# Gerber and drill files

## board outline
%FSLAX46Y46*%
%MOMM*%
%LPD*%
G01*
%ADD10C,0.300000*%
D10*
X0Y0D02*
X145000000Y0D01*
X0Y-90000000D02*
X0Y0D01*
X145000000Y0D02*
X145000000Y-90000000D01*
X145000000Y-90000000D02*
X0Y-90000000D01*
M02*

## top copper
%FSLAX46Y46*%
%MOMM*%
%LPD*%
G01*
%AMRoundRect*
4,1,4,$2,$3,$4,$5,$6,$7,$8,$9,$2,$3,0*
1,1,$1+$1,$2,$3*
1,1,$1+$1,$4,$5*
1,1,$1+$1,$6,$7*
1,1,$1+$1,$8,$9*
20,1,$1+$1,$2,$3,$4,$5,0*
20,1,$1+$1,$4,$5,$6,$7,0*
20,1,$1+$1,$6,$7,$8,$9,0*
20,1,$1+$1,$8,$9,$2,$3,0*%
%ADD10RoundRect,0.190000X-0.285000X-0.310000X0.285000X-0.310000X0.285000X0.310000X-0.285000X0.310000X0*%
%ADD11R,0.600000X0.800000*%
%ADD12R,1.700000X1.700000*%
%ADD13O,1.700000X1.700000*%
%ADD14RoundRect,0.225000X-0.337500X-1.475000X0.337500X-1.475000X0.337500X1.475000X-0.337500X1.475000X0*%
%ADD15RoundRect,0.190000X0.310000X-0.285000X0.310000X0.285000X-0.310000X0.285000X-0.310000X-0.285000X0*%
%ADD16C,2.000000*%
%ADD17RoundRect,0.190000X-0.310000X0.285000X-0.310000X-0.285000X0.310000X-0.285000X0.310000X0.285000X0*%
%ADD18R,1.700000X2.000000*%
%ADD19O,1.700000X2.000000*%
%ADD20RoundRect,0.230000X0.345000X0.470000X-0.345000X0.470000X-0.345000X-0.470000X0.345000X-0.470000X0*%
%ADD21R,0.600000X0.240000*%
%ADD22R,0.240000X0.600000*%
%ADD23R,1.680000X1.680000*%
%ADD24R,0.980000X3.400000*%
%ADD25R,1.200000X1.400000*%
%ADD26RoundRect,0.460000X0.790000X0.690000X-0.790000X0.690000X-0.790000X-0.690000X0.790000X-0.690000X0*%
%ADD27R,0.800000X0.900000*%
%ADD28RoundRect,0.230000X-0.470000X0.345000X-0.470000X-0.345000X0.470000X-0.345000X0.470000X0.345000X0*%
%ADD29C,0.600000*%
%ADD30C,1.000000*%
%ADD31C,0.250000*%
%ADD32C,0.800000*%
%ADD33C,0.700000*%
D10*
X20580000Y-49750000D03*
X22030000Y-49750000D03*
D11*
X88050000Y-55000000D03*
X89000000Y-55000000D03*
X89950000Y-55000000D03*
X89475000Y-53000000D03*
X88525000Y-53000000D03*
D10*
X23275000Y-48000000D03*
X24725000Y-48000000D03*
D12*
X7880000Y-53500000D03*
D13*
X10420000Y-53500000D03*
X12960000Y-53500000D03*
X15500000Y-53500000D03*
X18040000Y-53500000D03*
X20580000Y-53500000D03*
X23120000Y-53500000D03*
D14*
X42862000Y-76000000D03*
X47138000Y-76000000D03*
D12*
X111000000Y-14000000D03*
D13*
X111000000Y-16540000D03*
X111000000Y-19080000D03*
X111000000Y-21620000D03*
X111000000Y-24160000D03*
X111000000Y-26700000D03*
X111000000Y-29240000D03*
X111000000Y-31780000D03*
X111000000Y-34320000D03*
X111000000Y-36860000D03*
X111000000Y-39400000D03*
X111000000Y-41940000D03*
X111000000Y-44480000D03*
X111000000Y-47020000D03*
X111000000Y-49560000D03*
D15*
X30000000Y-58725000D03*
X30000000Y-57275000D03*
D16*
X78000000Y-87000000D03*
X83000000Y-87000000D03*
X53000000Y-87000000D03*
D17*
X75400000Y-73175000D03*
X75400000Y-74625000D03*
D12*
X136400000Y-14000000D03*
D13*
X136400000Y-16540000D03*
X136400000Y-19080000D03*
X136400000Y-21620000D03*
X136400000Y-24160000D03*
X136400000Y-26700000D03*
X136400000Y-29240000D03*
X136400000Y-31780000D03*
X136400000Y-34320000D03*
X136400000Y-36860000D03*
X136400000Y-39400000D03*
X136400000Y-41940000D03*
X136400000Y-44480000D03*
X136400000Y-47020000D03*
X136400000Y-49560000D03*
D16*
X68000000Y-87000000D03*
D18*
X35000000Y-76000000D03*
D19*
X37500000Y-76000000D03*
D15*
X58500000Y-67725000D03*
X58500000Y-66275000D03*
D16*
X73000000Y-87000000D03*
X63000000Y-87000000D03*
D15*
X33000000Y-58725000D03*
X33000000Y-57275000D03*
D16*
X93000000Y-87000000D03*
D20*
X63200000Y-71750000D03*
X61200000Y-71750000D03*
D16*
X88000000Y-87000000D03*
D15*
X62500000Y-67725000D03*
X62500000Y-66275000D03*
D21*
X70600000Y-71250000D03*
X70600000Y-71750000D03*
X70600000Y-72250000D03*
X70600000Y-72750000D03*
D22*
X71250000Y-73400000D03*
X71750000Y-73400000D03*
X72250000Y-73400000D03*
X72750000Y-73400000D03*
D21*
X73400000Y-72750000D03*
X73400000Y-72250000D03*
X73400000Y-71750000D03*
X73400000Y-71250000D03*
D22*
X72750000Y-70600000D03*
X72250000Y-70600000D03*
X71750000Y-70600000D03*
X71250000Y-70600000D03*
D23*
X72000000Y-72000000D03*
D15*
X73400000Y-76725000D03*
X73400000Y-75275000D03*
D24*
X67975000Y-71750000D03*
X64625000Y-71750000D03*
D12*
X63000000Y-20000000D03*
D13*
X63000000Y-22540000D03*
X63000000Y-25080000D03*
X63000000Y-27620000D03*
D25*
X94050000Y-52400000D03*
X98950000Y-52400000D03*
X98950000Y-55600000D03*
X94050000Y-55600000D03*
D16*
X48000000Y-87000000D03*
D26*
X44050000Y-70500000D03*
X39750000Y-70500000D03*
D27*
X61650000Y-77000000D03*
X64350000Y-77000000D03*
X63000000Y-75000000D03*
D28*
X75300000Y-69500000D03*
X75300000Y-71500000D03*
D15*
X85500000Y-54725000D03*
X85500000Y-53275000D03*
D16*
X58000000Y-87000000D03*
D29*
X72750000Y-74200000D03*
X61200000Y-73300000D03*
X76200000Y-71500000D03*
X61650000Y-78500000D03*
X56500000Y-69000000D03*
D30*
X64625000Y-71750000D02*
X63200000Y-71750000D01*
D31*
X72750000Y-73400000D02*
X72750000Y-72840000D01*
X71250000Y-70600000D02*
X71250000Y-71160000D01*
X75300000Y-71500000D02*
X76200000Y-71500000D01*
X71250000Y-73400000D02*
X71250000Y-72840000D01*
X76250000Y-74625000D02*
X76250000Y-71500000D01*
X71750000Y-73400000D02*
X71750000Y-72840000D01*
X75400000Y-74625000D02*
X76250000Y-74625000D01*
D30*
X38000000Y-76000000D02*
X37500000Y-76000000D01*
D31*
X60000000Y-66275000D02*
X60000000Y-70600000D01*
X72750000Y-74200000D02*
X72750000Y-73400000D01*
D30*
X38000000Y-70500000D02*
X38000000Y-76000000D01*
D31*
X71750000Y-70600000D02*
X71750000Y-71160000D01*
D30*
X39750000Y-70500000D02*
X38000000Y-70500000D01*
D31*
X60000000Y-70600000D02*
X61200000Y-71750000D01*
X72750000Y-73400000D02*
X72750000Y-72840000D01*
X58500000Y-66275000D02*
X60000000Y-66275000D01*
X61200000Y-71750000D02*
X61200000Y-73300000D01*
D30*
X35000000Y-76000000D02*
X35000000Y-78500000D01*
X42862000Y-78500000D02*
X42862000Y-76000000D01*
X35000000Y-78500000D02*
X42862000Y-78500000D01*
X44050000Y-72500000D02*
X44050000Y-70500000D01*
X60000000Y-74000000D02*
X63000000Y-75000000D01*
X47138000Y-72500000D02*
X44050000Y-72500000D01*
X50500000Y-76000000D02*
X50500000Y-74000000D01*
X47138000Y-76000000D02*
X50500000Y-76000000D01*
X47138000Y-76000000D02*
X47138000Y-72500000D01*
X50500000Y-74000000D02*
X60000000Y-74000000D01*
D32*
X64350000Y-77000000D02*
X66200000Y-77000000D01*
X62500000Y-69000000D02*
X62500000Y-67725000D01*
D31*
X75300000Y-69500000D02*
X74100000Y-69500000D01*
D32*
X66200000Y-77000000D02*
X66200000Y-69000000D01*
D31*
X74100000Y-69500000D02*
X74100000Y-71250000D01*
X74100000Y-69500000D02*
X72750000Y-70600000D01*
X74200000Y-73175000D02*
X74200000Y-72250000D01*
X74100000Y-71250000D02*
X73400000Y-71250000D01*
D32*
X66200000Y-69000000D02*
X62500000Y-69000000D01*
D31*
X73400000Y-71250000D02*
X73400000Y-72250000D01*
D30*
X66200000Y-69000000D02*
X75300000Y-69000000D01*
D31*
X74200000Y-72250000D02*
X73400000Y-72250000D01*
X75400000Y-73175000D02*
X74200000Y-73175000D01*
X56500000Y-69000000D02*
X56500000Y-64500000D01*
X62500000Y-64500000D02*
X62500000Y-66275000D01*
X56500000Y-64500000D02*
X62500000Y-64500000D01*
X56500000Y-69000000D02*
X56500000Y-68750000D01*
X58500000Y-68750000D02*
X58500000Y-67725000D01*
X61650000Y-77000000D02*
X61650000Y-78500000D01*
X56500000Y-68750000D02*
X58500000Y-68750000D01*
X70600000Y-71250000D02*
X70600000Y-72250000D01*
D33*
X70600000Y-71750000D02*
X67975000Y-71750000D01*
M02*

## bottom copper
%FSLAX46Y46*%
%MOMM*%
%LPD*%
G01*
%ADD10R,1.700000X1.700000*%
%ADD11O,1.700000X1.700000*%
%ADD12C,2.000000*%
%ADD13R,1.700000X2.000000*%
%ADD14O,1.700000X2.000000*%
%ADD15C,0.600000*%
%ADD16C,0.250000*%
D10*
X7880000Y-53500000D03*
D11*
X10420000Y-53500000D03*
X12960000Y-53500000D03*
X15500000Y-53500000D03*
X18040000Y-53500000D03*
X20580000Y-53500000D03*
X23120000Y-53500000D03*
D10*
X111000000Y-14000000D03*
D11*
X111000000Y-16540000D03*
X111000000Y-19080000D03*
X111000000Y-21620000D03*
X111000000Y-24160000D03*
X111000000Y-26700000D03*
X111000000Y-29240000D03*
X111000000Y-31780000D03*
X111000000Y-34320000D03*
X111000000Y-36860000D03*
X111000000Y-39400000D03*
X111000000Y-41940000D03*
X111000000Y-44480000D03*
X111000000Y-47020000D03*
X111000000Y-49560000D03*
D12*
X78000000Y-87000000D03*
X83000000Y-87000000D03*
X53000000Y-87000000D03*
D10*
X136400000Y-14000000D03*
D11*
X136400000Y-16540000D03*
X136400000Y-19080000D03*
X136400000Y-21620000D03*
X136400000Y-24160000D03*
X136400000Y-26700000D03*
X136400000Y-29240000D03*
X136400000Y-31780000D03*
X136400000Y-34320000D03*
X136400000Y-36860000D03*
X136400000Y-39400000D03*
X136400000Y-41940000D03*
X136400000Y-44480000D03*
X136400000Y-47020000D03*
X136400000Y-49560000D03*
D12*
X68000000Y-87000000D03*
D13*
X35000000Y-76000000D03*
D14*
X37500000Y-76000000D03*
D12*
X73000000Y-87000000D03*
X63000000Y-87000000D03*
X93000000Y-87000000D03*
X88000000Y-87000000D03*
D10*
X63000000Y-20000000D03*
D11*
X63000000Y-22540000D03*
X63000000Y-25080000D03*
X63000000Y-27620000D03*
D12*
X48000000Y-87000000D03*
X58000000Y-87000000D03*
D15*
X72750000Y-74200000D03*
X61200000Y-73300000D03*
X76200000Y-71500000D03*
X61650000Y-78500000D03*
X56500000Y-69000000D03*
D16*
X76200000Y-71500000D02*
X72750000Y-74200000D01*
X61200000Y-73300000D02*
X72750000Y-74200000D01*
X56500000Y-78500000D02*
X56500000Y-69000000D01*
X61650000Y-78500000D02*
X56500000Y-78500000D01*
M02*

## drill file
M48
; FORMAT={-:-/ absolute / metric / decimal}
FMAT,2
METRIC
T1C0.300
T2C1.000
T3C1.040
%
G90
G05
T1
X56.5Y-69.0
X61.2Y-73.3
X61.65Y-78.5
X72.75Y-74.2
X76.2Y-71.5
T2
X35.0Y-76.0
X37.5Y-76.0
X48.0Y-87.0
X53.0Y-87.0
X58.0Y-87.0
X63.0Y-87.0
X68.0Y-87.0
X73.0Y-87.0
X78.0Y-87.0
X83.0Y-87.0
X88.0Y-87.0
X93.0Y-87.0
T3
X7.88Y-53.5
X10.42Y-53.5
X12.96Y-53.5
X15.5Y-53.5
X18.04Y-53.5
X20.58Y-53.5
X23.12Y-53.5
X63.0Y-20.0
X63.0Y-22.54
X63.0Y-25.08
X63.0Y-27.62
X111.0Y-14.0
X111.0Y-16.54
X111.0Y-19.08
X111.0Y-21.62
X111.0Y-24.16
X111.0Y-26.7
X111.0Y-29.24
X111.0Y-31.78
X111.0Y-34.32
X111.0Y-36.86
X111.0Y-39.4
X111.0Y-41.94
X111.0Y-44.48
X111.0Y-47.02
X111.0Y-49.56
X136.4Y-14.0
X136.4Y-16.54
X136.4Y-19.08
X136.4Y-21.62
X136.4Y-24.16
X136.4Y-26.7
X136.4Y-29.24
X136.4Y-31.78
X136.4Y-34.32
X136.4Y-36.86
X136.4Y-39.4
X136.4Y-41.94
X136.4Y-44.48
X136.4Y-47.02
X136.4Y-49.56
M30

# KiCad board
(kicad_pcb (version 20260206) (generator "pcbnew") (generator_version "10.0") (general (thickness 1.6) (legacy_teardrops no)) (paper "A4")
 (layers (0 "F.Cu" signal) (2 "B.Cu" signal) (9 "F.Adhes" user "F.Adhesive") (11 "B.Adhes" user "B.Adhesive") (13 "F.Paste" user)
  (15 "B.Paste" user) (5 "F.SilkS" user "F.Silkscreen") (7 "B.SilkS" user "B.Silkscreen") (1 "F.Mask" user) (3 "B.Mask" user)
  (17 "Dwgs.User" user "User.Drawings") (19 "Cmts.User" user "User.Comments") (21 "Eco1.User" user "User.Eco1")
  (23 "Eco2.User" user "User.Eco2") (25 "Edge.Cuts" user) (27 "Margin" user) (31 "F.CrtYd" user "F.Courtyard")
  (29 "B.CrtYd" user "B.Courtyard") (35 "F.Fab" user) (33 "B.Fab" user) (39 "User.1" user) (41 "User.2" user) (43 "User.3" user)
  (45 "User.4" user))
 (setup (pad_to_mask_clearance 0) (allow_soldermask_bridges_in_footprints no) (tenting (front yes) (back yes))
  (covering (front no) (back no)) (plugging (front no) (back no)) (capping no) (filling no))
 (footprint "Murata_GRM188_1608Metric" (layer "F.Cu") (at 21.305 49.75)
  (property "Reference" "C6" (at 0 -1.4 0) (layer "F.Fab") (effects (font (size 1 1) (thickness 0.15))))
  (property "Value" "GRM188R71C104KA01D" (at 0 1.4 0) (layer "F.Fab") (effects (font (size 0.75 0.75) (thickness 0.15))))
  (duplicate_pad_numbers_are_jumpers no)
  (pad "1" smd roundrect (at -0.725 0) (size 0.95 1) (layers "F.Cu" "F.Mask" "F.Paste") (roundrect_rratio 0.2) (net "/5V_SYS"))
  (pad "2" smd roundrect (at 0.725 0) (size 0.95 1) (layers "F.Cu" "F.Mask" "F.Paste") (roundrect_rratio 0.2) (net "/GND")))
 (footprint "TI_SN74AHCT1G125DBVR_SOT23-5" (layer "F.Cu") (at 89 54)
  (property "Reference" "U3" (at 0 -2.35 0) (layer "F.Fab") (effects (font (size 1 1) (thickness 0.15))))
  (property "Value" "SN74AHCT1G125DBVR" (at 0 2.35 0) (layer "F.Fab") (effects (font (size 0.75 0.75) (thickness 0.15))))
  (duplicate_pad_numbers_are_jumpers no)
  (pad "1" smd rect (at -0.95 1) (size 0.6 0.8) (layers "F.Cu" "F.Mask" "F.Paste") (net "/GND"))
  (pad "2" smd rect (at 0 1) (size 0.6 0.8) (layers "F.Cu" "F.Mask" "F.Paste") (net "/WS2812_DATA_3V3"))
  (pad "3" smd rect (at 0.95 1) (size 0.6 0.8) (layers "F.Cu" "F.Mask" "F.Paste") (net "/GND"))
  (pad "4" smd rect (at 0.475 -1) (size 0.6 0.8) (layers "F.Cu" "F.Mask" "F.Paste") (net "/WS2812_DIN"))
  (pad "5" smd rect (at -0.475 -1) (size 0.6 0.8) (layers "F.Cu" "F.Mask" "F.Paste") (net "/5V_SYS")))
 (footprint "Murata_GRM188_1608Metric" (layer "F.Cu") (at 24 48)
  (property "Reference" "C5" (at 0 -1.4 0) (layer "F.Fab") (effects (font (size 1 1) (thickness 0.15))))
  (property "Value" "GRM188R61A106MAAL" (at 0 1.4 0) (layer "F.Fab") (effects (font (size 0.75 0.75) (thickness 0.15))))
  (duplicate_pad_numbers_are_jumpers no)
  (pad "1" smd roundrect (at -0.725 0) (size 0.95 1) (layers "F.Cu" "F.Mask" "F.Paste") (roundrect_rratio 0.2) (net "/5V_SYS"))
  (pad "2" smd roundrect (at 0.725 0) (size 0.95 1) (layers "F.Cu" "F.Mask" "F.Paste") (roundrect_rratio 0.2) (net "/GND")))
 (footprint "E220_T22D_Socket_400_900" (layer "F.Cu") (at 5 52)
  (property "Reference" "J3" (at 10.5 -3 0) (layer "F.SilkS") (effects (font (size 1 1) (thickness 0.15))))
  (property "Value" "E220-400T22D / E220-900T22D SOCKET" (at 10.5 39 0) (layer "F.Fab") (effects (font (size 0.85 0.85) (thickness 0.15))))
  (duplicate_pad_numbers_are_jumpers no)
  (pad "1" thru_hole rect (at 2.88 1.5) (size 1.7 1.7) (drill 1.04) (layers "*.Cu" "*.Mask") (remove_unused_layers no) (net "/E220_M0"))
  (pad "2" thru_hole oval (at 5.42 1.5) (size 1.7 1.7) (drill 1.04) (layers "*.Cu" "*.Mask") (remove_unused_layers no) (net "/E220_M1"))
  (pad "3" thru_hole oval (at 7.96 1.5) (size 1.7 1.7) (drill 1.04) (layers "*.Cu" "*.Mask") (remove_unused_layers no) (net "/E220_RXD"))
  (pad "4" thru_hole oval (at 10.5 1.5) (size 1.7 1.7) (drill 1.04) (layers "*.Cu" "*.Mask") (remove_unused_layers no) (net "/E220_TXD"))
  (pad "5" thru_hole oval (at 13.04 1.5) (size 1.7 1.7) (drill 1.04) (layers "*.Cu" "*.Mask") (remove_unused_layers no) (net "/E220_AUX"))
  (pad "6" thru_hole oval (at 15.58 1.5) (size 1.7 1.7) (drill 1.04) (layers "*.Cu" "*.Mask") (remove_unused_layers no) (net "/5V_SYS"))
  (pad "7" thru_hole oval (at 18.12 1.5) (size 1.7 1.7) (drill 1.04) (layers "*.Cu" "*.Mask") (remove_unused_layers no) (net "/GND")))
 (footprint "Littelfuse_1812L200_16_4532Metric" (layer "F.Cu") (at 45 76)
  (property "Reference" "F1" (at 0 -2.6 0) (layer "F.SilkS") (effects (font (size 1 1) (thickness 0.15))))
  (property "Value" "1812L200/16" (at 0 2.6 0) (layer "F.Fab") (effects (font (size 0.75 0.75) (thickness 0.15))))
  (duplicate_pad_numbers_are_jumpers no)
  (pad "1" smd roundrect (at -2.138 0) (size 1.125 3.4) (layers "F.Cu" "F.Mask" "F.Paste") (roundrect_rratio 0.2) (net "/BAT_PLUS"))
  (pad "2" smd roundrect (at 2.138 0) (size 1.125 3.4) (layers "F.Cu" "F.Mask" "F.Paste") (roundrect_rratio 0.2) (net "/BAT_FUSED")))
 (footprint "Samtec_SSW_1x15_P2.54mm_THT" (layer "F.Cu") (at 111 14)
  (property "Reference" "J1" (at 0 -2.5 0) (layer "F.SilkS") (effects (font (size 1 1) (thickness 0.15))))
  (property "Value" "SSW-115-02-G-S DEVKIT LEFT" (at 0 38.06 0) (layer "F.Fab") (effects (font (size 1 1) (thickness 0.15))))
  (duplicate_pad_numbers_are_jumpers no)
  (pad "1" thru_hole rect (at 0 0) (size 1.7 1.7) (drill 1.04) (layers "*.Cu" "*.Mask") (remove_unused_layers no) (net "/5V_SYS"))
  (pad "2" thru_hole oval (at 0 2.54) (size 1.7 1.7) (drill 1.04) (layers "*.Cu" "*.Mask") (remove_unused_layers no) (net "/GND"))
  (pad "3" thru_hole oval (at 0 5.08) (size 1.7 1.7) (drill 1.04) (layers "*.Cu" "*.Mask") (remove_unused_layers no))
  (pad "4" thru_hole oval (at 0 7.62) (size 1.7 1.7) (drill 1.04) (layers "*.Cu" "*.Mask") (remove_unused_layers no))
  (pad "5" thru_hole oval (at 0 10.16) (size 1.7 1.7) (drill 1.04) (layers "*.Cu" "*.Mask") (remove_unused_layers no))
  (pad "6" thru_hole oval (at 0 12.7) (size 1.7 1.7) (drill 1.04) (layers "*.Cu" "*.Mask") (remove_unused_layers no) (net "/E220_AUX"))
  (pad "7" thru_hole oval (at 0 15.24) (size 1.7 1.7) (drill 1.04) (layers "*.Cu" "*.Mask") (remove_unused_layers no) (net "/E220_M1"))
  (pad "8" thru_hole oval (at 0 17.78) (size 1.7 1.7) (drill 1.04) (layers "*.Cu" "*.Mask") (remove_unused_layers no) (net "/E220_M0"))
  (pad "9" thru_hole oval (at 0 20.32) (size 1.7 1.7) (drill 1.04) (layers "*.Cu" "*.Mask") (remove_unused_layers no))
  (pad "10" thru_hole oval (at 0 22.86) (size 1.7 1.7) (drill 1.04) (layers "*.Cu" "*.Mask") (remove_unused_layers no))
  (pad "11" thru_hole oval (at 0 25.4) (size 1.7 1.7) (drill 1.04) (layers "*.Cu" "*.Mask") (remove_unused_layers no))
  (pad "12" thru_hole oval (at 0 27.94) (size 1.7 1.7) (drill 1.04) (layers "*.Cu" "*.Mask") (remove_unused_layers no))
  (pad "13" thru_hole oval (at 0 30.48) (size 1.7 1.7) (drill 1.04) (layers "*.Cu" "*.Mask") (remove_unused_layers no))
  (pad "14" thru_hole oval (at 0 33.02) (size 1.7 1.7) (drill 1.04) (layers "*.Cu" "*.Mask") (remove_unused_layers no))
  (pad "15" thru_hole oval (at 0 35.56) (size 1.7 1.7) (drill 1.04) (layers "*.Cu" "*.Mask") (remove_unused_layers no)))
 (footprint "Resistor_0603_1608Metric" (layer "F.Cu") (at 30 58 90)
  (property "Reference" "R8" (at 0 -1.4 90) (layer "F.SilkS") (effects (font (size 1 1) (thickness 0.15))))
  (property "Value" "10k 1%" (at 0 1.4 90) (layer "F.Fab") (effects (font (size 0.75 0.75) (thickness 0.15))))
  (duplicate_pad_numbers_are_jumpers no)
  (pad "1" smd roundrect (at -0.725 0 90) (size 0.95 1) (layers "F.Cu" "F.Mask" "F.Paste") (roundrect_rratio 0.2) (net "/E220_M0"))
  (pad "2" smd roundrect (at 0.725 0 90) (size 0.95 1) (layers "F.Cu" "F.Mask" "F.Paste") (roundrect_rratio 0.2) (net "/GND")))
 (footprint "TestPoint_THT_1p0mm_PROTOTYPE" (layer "F.Cu") (at 78 87)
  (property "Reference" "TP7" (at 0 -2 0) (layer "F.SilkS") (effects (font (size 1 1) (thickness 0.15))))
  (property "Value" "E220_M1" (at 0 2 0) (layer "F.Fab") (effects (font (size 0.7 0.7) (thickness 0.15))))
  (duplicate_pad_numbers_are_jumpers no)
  (pad "1" thru_hole circle (at 0 0) (size 2 2) (drill 1) (layers "*.Cu" "*.Mask") (remove_unused_layers no) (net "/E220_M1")))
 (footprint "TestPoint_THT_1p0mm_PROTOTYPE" (layer "F.Cu") (at 83 87)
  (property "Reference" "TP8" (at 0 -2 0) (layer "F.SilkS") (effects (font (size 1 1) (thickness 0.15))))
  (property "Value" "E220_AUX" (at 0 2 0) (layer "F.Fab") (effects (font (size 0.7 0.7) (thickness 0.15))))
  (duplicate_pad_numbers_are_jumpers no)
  (pad "1" thru_hole circle (at 0 0) (size 2 2) (drill 1) (layers "*.Cu" "*.Mask") (remove_unused_layers no) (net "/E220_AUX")))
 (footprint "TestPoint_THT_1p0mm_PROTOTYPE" (layer "F.Cu") (at 53 87)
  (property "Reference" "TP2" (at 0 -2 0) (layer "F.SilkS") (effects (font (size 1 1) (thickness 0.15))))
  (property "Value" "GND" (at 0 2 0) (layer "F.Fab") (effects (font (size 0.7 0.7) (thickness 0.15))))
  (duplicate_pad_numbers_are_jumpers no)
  (pad "1" thru_hole circle (at 0 0) (size 2 2) (drill 1) (layers "*.Cu" "*.Mask") (remove_unused_layers no) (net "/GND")))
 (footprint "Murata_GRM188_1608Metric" (layer "F.Cu") (at 75.4 73.9 -90)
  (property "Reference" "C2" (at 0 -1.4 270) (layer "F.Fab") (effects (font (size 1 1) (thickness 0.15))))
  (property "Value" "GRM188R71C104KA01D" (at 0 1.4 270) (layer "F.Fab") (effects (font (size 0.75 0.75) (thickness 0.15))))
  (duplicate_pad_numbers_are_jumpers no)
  (pad "1" smd roundrect (at -0.725 0 270) (size 0.95 1) (layers "F.Cu" "F.Mask" "F.Paste") (roundrect_rratio 0.2) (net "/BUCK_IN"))
  (pad "2" smd roundrect (at 0.725 0 270) (size 0.95 1) (layers "F.Cu" "F.Mask" "F.Paste") (roundrect_rratio 0.2) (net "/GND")))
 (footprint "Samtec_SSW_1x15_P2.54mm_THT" (layer "F.Cu") (at 136.4 14)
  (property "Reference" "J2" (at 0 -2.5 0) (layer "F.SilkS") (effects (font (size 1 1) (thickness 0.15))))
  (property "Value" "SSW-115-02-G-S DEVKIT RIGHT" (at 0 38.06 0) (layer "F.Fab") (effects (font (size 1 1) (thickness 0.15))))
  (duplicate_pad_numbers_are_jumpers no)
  (pad "1" thru_hole rect (at 0 0) (size 1.7 1.7) (drill 1.04) (layers "*.Cu" "*.Mask") (remove_unused_layers no) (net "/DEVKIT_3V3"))
  (pad "2" thru_hole oval (at 0 2.54) (size 1.7 1.7) (drill 1.04) (layers "*.Cu" "*.Mask") (remove_unused_layers no) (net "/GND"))
  (pad "3" thru_hole oval (at 0 5.08) (size 1.7 1.7) (drill 1.04) (layers "*.Cu" "*.Mask") (remove_unused_layers no))
  (pad "4" thru_hole oval (at 0 7.62) (size 1.7 1.7) (drill 1.04) (layers "*.Cu" "*.Mask") (remove_unused_layers no))
  (pad "5" thru_hole oval (at 0 10.16) (size 1.7 1.7) (drill 1.04) (layers "*.Cu" "*.Mask") (remove_unused_layers no)
   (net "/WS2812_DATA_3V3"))
  (pad "6" thru_hole oval (at 0 12.7) (size 1.7 1.7) (drill 1.04) (layers "*.Cu" "*.Mask") (remove_unused_layers no) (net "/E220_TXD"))
  (pad "7" thru_hole oval (at 0 15.24) (size 1.7 1.7) (drill 1.04) (layers "*.Cu" "*.Mask") (remove_unused_layers no) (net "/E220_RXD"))
  (pad "8" thru_hole oval (at 0 17.78) (size 1.7 1.7) (drill 1.04) (layers "*.Cu" "*.Mask") (remove_unused_layers no))
  (pad "9" thru_hole oval (at 0 20.32) (size 1.7 1.7) (drill 1.04) (layers "*.Cu" "*.Mask") (remove_unused_layers no))
  (pad "10" thru_hole oval (at 0 22.86) (size 1.7 1.7) (drill 1.04) (layers "*.Cu" "*.Mask") (remove_unused_layers no))
  (pad "11" thru_hole oval (at 0 25.4) (size 1.7 1.7) (drill 1.04) (layers "*.Cu" "*.Mask") (remove_unused_layers no) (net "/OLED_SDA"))
  (pad "12" thru_hole oval (at 0 27.94) (size 1.7 1.7) (drill 1.04) (layers "*.Cu" "*.Mask") (remove_unused_layers no))
  (pad "13" thru_hole oval (at 0 30.48) (size 1.7 1.7) (drill 1.04) (layers "*.Cu" "*.Mask") (remove_unused_layers no))
  (pad "14" thru_hole oval (at 0 33.02) (size 1.7 1.7) (drill 1.04) (layers "*.Cu" "*.Mask") (remove_unused_layers no) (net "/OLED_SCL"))
  (pad "15" thru_hole oval (at 0 35.56) (size 1.7 1.7) (drill 1.04) (layers "*.Cu" "*.Mask") (remove_unused_layers no)))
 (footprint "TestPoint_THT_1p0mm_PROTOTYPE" (layer "F.Cu") (at 68 87)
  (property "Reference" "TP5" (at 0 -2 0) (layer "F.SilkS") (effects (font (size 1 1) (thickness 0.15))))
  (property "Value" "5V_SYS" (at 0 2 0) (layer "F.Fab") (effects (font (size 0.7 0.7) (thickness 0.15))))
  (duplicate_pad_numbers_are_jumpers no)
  (pad "1" thru_hole circle (at 0 0) (size 2 2) (drill 1) (layers "*.Cu" "*.Mask") (remove_unused_layers no) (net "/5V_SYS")))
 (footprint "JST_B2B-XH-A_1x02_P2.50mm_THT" (layer "F.Cu") (at 35 76)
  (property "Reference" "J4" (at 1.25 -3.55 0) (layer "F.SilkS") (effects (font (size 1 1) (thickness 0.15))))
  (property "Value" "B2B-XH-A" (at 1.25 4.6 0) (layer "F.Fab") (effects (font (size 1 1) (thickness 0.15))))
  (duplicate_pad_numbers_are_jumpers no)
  (pad "1" thru_hole rect (at 0 0) (size 1.7 2) (drill 1) (layers "*.Cu" "*.Mask") (remove_unused_layers no) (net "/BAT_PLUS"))
  (pad "2" thru_hole oval (at 2.5 0) (size 1.7 2) (drill 1) (layers "*.Cu" "*.Mask") (remove_unused_layers no) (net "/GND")))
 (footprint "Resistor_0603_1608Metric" (layer "F.Cu") (at 58.5 67 90)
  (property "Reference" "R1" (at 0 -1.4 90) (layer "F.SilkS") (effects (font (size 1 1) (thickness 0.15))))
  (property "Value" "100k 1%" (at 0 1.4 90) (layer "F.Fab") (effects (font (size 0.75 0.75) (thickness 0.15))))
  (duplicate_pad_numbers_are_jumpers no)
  (pad "1" smd roundrect (at -0.725 0 90) (size 0.95 1) (layers "F.Cu" "F.Mask" "F.Paste") (roundrect_rratio 0.2) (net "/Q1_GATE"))
  (pad "2" smd roundrect (at 0.725 0 90) (size 0.95 1) (layers "F.Cu" "F.Mask" "F.Paste") (roundrect_rratio 0.2) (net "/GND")))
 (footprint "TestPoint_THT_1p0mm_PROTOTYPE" (layer "F.Cu") (at 73 87)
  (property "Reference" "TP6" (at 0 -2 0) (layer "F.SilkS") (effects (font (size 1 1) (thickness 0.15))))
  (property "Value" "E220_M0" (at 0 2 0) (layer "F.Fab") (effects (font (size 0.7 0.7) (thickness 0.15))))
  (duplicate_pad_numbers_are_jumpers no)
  (pad "1" thru_hole circle (at 0 0) (size 2 2) (drill 1) (layers "*.Cu" "*.Mask") (remove_unused_layers no) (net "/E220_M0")))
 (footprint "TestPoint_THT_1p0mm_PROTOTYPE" (layer "F.Cu") (at 63 87)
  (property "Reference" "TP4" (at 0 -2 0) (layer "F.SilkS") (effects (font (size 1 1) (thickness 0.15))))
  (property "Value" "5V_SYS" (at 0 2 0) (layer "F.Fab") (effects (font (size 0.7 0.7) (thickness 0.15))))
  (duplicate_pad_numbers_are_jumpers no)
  (pad "1" thru_hole circle (at 0 0) (size 2 2) (drill 1) (layers "*.Cu" "*.Mask") (remove_unused_layers no) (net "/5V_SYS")))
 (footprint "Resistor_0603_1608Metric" (layer "F.Cu") (at 33 58 90)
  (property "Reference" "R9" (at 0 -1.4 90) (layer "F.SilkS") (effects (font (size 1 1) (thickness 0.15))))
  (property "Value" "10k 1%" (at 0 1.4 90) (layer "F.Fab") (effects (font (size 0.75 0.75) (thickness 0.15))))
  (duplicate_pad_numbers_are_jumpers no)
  (pad "1" smd roundrect (at -0.725 0 90) (size 0.95 1) (layers "F.Cu" "F.Mask" "F.Paste") (roundrect_rratio 0.2) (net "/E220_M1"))
  (pad "2" smd roundrect (at 0.725 0 90) (size 0.95 1) (layers "F.Cu" "F.Mask" "F.Paste") (roundrect_rratio 0.2) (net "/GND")))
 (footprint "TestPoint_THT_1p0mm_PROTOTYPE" (layer "F.Cu") (at 93 87)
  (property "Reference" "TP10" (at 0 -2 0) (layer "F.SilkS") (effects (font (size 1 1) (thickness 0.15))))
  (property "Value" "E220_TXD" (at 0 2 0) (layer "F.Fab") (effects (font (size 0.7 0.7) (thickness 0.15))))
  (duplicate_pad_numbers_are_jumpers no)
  (pad "1" thru_hole circle (at 0 0) (size 2 2) (drill 1) (layers "*.Cu" "*.Mask") (remove_unused_layers no) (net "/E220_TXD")))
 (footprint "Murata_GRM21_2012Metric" (layer "F.Cu") (at 62.2 71.75 180)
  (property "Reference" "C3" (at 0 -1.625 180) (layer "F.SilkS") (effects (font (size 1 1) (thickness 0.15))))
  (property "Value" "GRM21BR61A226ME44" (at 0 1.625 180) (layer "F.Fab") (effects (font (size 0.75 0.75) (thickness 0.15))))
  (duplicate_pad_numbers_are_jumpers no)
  (pad "1" smd roundrect (at -1 0 180) (size 1.15 1.4) (layers "F.Cu" "F.Mask" "F.Paste") (roundrect_rratio 0.2) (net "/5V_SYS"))
  (pad "2" smd roundrect (at 1 0 180) (size 1.15 1.4) (layers "F.Cu" "F.Mask" "F.Paste") (roundrect_rratio 0.2) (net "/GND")))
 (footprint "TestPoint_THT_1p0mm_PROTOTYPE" (layer "F.Cu") (at 88 87)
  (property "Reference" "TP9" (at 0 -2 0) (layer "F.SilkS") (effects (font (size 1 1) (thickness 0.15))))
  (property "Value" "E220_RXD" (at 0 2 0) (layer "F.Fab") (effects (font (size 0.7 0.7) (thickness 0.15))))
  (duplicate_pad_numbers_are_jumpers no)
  (pad "1" thru_hole circle (at 0 0) (size 2 2) (drill 1) (layers "*.Cu" "*.Mask") (remove_unused_layers no) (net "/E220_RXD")))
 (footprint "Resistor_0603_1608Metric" (layer "F.Cu") (at 62.5 67 90)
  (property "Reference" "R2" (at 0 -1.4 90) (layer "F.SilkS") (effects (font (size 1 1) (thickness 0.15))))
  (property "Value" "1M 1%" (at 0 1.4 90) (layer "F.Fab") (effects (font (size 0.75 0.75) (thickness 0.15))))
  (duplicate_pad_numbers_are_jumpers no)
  (pad "1" smd roundrect (at -0.725 0 90) (size 0.95 1) (layers "F.Cu" "F.Mask" "F.Paste") (roundrect_rratio 0.2) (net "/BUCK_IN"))
  (pad "2" smd roundrect (at 0.725 0 90) (size 0.95 1) (layers "F.Cu" "F.Mask" "F.Paste") (roundrect_rratio 0.2) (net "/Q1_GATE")))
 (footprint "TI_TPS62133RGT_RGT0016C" (layer "F.Cu") (at 72 72)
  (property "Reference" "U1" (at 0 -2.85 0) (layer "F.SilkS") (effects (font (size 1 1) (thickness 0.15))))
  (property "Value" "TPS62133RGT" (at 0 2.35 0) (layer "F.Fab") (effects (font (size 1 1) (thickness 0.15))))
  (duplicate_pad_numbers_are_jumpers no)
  (pad "" smd rect (at 0 0) (size 1.55 1.55) (layers "F.Paste"))
  (pad "1" smd rect (at -1.4 -0.75) (size 0.6 0.24) (layers "F.Cu" "F.Mask" "F.Paste") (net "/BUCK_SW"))
  (pad "2" smd rect (at -1.4 -0.25) (size 0.6 0.24) (layers "F.Cu" "F.Mask" "F.Paste") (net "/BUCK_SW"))
  (pad "3" smd rect (at -1.4 0.25) (size 0.6 0.24) (layers "F.Cu" "F.Mask" "F.Paste") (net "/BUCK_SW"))
  (pad "4" smd rect (at -1.4 0.75) (size 0.6 0.24) (layers "F.Cu" "F.Mask" "F.Paste"))
  (pad "5" smd rect (at -0.75 1.4) (size 0.24 0.6) (layers "F.Cu" "F.Mask" "F.Paste") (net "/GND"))
  (pad "6" smd rect (at -0.25 1.4) (size 0.24 0.6) (layers "F.Cu" "F.Mask" "F.Paste") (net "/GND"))
  (pad "7" smd rect (at 0.25 1.4) (size 0.24 0.6) (layers "F.Cu" "F.Mask" "F.Paste") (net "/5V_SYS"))
  (pad "8" smd rect (at 0.75 1.4) (size 0.24 0.6) (layers "F.Cu" "F.Mask" "F.Paste") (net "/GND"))
  (pad "9" smd rect (at 1.4 0.75) (size 0.6 0.24) (layers "F.Cu" "F.Mask" "F.Paste") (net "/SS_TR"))
  (pad "10" smd rect (at 1.4 0.25) (size 0.6 0.24) (layers "F.Cu" "F.Mask" "F.Paste") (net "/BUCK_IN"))
  (pad "11" smd rect (at 1.4 -0.25) (size 0.6 0.24) (layers "F.Cu" "F.Mask" "F.Paste") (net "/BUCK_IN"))
  (pad "12" smd rect (at 1.4 -0.75) (size 0.6 0.24) (layers "F.Cu" "F.Mask" "F.Paste") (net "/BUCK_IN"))
  (pad "13" smd rect (at 0.75 -1.4) (size 0.24 0.6) (layers "F.Cu" "F.Mask" "F.Paste") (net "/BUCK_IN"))
  (pad "14" smd rect (at 0.25 -1.4) (size 0.24 0.6) (layers "F.Cu" "F.Mask" "F.Paste") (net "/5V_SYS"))
  (pad "15" smd rect (at -0.25 -1.4) (size 0.24 0.6) (layers "F.Cu" "F.Mask" "F.Paste") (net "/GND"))
  (pad "16" smd rect (at -0.75 -1.4) (size 0.24 0.6) (layers "F.Cu" "F.Mask" "F.Paste") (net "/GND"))
  (pad "EP" smd rect (at 0 0) (size 1.68 1.68) (layers "F.Cu" "F.Mask") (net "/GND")))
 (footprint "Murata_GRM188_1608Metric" (layer "F.Cu") (at 73.4 76 90)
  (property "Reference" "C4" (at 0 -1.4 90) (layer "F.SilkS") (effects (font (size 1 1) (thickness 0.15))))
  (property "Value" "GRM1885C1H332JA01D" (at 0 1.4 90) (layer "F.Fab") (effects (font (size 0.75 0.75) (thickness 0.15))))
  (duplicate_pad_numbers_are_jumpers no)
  (pad "1" smd roundrect (at -0.725 0 90) (size 0.95 1) (layers "F.Cu" "F.Mask" "F.Paste") (roundrect_rratio 0.2) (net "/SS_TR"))
  (pad "2" smd roundrect (at 0.725 0 90) (size 0.95 1) (layers "F.Cu" "F.Mask" "F.Paste") (roundrect_rratio 0.2) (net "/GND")))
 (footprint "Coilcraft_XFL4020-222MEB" (layer "F.Cu") (at 66.3 71.75 180)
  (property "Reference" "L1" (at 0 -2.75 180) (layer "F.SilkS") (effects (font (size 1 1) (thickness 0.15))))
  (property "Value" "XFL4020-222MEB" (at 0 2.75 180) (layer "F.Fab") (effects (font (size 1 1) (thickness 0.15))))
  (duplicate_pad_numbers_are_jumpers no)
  (pad "1" smd rect (at -1.675 0 180) (size 0.98 3.4) (layers "F.Cu" "F.Mask" "F.Paste") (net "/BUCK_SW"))
  (pad "2" smd rect (at 1.675 0 180) (size 0.98 3.4) (layers "F.Cu" "F.Mask" "F.Paste") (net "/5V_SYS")))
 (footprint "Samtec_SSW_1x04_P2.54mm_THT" (layer "F.Cu") (at 63 20)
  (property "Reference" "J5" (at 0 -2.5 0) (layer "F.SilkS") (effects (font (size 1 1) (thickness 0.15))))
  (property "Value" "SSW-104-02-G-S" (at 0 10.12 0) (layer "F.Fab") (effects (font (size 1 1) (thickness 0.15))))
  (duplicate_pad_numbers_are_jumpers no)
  (pad "1" thru_hole rect (at 0 0) (size 1.7 1.7) (drill 1.04) (layers "*.Cu" "*.Mask") (remove_unused_layers no) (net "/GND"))
  (pad "2" thru_hole oval (at 0 2.54) (size 1.7 1.7) (drill 1.04) (layers "*.Cu" "*.Mask") (remove_unused_layers no) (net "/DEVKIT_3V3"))
  (pad "3" thru_hole oval (at 0 5.08) (size 1.7 1.7) (drill 1.04) (layers "*.Cu" "*.Mask") (remove_unused_layers no) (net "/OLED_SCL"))
  (pad "4" thru_hole oval (at 0 7.62) (size 1.7 1.7) (drill 1.04) (layers "*.Cu" "*.Mask") (remove_unused_layers no) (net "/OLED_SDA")))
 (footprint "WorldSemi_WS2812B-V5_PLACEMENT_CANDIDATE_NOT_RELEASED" (layer "F.Cu") (at 96.5 54)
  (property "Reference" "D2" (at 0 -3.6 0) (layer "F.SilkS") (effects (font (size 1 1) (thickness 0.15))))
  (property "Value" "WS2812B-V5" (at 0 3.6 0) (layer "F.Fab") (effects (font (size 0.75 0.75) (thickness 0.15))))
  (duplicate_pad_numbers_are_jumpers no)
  (pad "1" smd rect (at -2.45 -1.6) (size 1.2 1.4) (layers "F.Cu" "F.Mask" "F.Paste") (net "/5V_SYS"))
  (pad "2" smd rect (at 2.45 -1.6) (size 1.2 1.4) (layers "F.Cu" "F.Mask" "F.Paste"))
  (pad "3" smd rect (at 2.45 1.6) (size 1.2 1.4) (layers "F.Cu" "F.Mask" "F.Paste") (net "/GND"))
  (pad "4" smd rect (at -2.45 1.6) (size 1.2 1.4) (layers "F.Cu" "F.Mask" "F.Paste") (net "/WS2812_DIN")))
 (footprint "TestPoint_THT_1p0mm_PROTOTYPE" (layer "F.Cu") (at 48 87)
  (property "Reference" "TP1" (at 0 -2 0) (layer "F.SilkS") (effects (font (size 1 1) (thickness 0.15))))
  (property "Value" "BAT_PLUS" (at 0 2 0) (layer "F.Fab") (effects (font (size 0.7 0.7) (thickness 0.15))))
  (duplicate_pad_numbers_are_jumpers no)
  (pad "1" thru_hole circle (at 0 0) (size 2 2) (drill 1) (layers "*.Cu" "*.Mask") (remove_unused_layers no) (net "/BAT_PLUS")))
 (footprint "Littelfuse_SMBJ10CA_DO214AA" (layer "F.Cu") (at 41.9 70.5 180)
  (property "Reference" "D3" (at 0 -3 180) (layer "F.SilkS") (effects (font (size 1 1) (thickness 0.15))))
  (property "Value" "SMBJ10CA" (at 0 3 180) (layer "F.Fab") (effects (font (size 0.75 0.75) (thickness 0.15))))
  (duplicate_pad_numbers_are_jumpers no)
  (pad "1" smd roundrect (at -2.15 0 180) (size 2.5 2.3) (layers "F.Cu" "F.Mask" "F.Paste") (roundrect_rratio 0.2) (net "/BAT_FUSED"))
  (pad "2" smd roundrect (at 2.15 0 180) (size 2.5 2.3) (layers "F.Cu" "F.Mask" "F.Paste") (roundrect_rratio 0.2) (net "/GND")))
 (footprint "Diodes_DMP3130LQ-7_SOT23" (layer "F.Cu") (at 63 76)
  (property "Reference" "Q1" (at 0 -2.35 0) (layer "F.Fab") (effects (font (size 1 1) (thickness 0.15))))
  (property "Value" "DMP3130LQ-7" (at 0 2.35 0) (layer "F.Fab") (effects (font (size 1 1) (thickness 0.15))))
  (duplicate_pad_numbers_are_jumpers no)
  (pad "1" smd rect (at -1.35 1) (size 0.8 0.9) (layers "F.Cu" "F.Mask" "F.Paste") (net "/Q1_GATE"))
  (pad "2" smd rect (at 1.35 1) (size 0.8 0.9) (layers "F.Cu" "F.Mask" "F.Paste") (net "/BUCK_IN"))
  (pad "3" smd rect (at 0 -1) (size 0.8 0.9) (layers "F.Cu" "F.Mask" "F.Paste") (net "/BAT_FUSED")))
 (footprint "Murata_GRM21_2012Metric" (layer "F.Cu") (at 75.3 70.5 -90)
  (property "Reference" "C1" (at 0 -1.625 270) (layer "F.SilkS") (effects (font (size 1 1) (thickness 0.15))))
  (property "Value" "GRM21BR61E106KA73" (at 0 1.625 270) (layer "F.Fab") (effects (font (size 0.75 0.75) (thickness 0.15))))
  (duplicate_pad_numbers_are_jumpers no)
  (pad "1" smd roundrect (at -1 0 270) (size 1.15 1.4) (layers "F.Cu" "F.Mask" "F.Paste") (roundrect_rratio 0.2) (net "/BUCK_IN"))
  (pad "2" smd roundrect (at 1 0 270) (size 1.15 1.4) (layers "F.Cu" "F.Mask" "F.Paste") (roundrect_rratio 0.2) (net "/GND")))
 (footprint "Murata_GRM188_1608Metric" (layer "F.Cu") (at 85.5 54 90)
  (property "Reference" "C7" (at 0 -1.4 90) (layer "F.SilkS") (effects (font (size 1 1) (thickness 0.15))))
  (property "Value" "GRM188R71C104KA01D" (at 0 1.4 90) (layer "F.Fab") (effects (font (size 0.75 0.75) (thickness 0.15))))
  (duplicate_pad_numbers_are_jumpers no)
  (pad "1" smd roundrect (at -0.725 0 90) (size 0.95 1) (layers "F.Cu" "F.Mask" "F.Paste") (roundrect_rratio 0.2) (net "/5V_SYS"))
  (pad "2" smd roundrect (at 0.725 0 90) (size 0.95 1) (layers "F.Cu" "F.Mask" "F.Paste") (roundrect_rratio 0.2) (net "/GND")))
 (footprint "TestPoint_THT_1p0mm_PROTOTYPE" (layer "F.Cu") (at 58 87)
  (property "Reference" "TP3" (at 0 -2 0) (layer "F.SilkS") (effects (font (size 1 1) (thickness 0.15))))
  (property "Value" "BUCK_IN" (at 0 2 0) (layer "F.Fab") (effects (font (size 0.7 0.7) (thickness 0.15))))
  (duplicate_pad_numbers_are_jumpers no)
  (pad "1" thru_hole circle (at 0 0) (size 2 2) (drill 1) (layers "*.Cu" "*.Mask") (remove_unused_layers no) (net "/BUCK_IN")))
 (gr_line (start 0 0) (end 145 0) (stroke (width 0.3) (type default)) (layer "Edge.Cuts"))
 (gr_line (start 0 90) (end 0 0) (stroke (width 0.3) (type default)) (layer "Edge.Cuts"))
 (gr_line (start 145 0) (end 145 90) (stroke (width 0.3) (type default)) (layer "Edge.Cuts"))
 (gr_line (start 145 90) (end 0 90) (stroke (width 0.3) (type default)) (layer "Edge.Cuts"))
 (segment (start 64.625 71.75) (end 63.2 71.75) (width 1) (layer "F.Cu") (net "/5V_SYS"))
 (segment (start 72.75 73.4) (end 72.75 72.84) (width 0.25) (layer "F.Cu") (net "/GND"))
 (segment (start 71.25 70.6) (end 71.25 71.16) (width 0.25) (layer "F.Cu") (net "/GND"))
 (segment (start 75.3 71.5) (end 76.2 71.5) (width 0.25) (layer "F.Cu") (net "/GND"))
 (segment (start 71.25 73.4) (end 71.25 72.84) (width 0.25) (layer "F.Cu") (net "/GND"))
 (segment (start 76.25 74.625) (end 76.25 71.5) (width 0.25) (layer "F.Cu") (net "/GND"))
 (segment (start 71.75 73.4) (end 71.75 72.84) (width 0.25) (layer "F.Cu") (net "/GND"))
 (segment (start 75.4 74.625) (end 76.25 74.625) (width 0.25) (layer "F.Cu") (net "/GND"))
 (segment (start 38 76) (end 37.5 76) (width 1) (layer "F.Cu") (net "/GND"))
 (segment (start 60 66.275) (end 60 70.6) (width 0.25) (layer "F.Cu") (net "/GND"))
 (segment (start 72.75 74.2) (end 72.75 73.4) (width 0.25) (layer "F.Cu") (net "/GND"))
 (segment (start 38 70.5) (end 38 76) (width 1) (layer "F.Cu") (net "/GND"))
 (segment (start 71.75 70.6) (end 71.75 71.16) (width 0.25) (layer "F.Cu") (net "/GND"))
 (segment (start 39.75 70.5) (end 38 70.5) (width 1) (layer "F.Cu") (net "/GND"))
 (segment (start 60 70.6) (end 61.2 71.75) (width 0.25) (layer "F.Cu") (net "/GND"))
 (segment (start 72.75 73.4) (end 72.75 72.84) (width 0.25) (layer "F.Cu") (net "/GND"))
 (segment (start 58.5 66.275) (end 60 66.275) (width 0.25) (layer "F.Cu") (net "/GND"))
 (segment (start 61.2 71.75) (end 61.2 73.3) (width 0.25) (layer "F.Cu") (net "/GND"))
 (via (at 72.75 74.2) (size 0.6) (drill 0.3) (layers "F.Cu" "B.Cu") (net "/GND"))
 (via (at 61.2 73.3) (size 0.6) (drill 0.3) (layers "F.Cu" "B.Cu") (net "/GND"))
 (via (at 76.2 71.5) (size 0.6) (drill 0.3) (layers "F.Cu" "B.Cu") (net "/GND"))
 (segment (start 76.2 71.5) (end 72.75 74.2) (width 0.25) (layer "B.Cu") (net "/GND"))
 (segment (start 61.2 73.3) (end 72.75 74.2) (width 0.25) (layer "B.Cu") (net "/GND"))
 (segment (start 35 76) (end 35 78.5) (width 1) (layer "F.Cu") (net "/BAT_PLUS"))
 (segment (start 42.862 78.5) (end 42.862 76) (width 1) (layer "F.Cu") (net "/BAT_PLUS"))
 (segment (start 35 78.5) (end 42.862 78.5) (width 1) (layer "F.Cu") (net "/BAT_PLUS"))
 (segment (start 44.05 72.5) (end 44.05 70.5) (width 1) (layer "F.Cu") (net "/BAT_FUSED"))
 (segment (start 60 74) (end 63 75) (width 1) (layer "F.Cu") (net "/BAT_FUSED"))
 (segment (start 47.138 72.5) (end 44.05 72.5) (width 1) (layer "F.Cu") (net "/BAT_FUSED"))
 (segment (start 50.5 76) (end 50.5 74) (width 1) (layer "F.Cu") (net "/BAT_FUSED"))
 (segment (start 47.138 76) (end 50.5 76) (width 1) (layer "F.Cu") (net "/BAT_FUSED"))
 (segment (start 47.138 76) (end 47.138 72.5) (width 1) (layer "F.Cu") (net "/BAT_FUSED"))
 (segment (start 50.5 74) (end 60 74) (width 1) (layer "F.Cu") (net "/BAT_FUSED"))
 (segment (start 64.35 77) (end 66.2 77) (width 0.8) (layer "F.Cu") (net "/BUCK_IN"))
 (segment (start 62.5 69) (end 62.5 67.725) (width 0.8) (layer "F.Cu") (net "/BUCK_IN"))
 (segment (start 75.3 69.5) (end 74.1 69.5) (width 0.25) (layer "F.Cu") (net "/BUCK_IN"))
 (segment (start 66.2 77) (end 66.2 69) (width 0.8) (layer "F.Cu") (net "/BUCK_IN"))
 (segment (start 74.1 69.5) (end 74.1 71.25) (width 0.25) (layer "F.Cu") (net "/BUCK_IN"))
 (segment (start 74.1 69.5) (end 72.75 70.6) (width 0.25) (layer "F.Cu") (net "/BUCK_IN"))
 (segment (start 74.2 73.175) (end 74.2 72.25) (width 0.25) (layer "F.Cu") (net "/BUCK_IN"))
 (segment (start 74.1 71.25) (end 73.4 71.25) (width 0.25) (layer "F.Cu") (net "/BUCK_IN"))
 (segment (start 66.2 69) (end 62.5 69) (width 0.8) (layer "F.Cu") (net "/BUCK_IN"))
 (segment (start 73.4 71.25) (end 73.4 72.25) (width 0.25) (layer "F.Cu") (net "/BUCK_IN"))
 (segment (start 66.2 69) (end 75.3 69) (width 1) (layer "F.Cu") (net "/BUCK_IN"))
 (segment (start 74.2 72.25) (end 73.4 72.25) (width 0.25) (layer "F.Cu") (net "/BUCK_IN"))
 (segment (start 75.4 73.175) (end 74.2 73.175) (width 0.25) (layer "F.Cu") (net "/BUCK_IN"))
 (segment (start 56.5 69) (end 56.5 64.5) (width 0.25) (layer "F.Cu") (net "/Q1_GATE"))
 (segment (start 62.5 64.5) (end 62.5 66.275) (width 0.25) (layer "F.Cu") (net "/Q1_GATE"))
 (segment (start 56.5 64.5) (end 62.5 64.5) (width 0.25) (layer "F.Cu") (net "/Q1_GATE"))
 (segment (start 56.5 69) (end 56.5 68.75) (width 0.25) (layer "F.Cu") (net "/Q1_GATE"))
 (segment (start 58.5 68.75) (end 58.5 67.725) (width 0.25) (layer "F.Cu") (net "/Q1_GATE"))
 (segment (start 61.65 77) (end 61.65 78.5) (width 0.25) (layer "F.Cu") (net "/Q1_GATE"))
 (segment (start 56.5 68.75) (end 58.5 68.75) (width 0.25) (layer "F.Cu") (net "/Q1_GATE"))
 (via (at 61.65 78.5) (size 0.6) (drill 0.3) (layers "F.Cu" "B.Cu") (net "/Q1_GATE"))
 (via (at 56.5 69) (size 0.6) (drill 0.3) (layers "F.Cu" "B.Cu") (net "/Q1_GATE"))
 (segment (start 56.5 78.5) (end 56.5 69) (width 0.25) (layer "B.Cu") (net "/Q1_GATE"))
 (segment (start 61.65 78.5) (end 56.5 78.5) (width 0.25) (layer "B.Cu") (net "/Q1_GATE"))
 (segment (start 70.6 71.25) (end 70.6 72.25) (width 0.25) (layer "F.Cu") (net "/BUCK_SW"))
 (segment (start 70.6 71.75) (end 67.975 71.75) (width 0.7) (layer "F.Cu") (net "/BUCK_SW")))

